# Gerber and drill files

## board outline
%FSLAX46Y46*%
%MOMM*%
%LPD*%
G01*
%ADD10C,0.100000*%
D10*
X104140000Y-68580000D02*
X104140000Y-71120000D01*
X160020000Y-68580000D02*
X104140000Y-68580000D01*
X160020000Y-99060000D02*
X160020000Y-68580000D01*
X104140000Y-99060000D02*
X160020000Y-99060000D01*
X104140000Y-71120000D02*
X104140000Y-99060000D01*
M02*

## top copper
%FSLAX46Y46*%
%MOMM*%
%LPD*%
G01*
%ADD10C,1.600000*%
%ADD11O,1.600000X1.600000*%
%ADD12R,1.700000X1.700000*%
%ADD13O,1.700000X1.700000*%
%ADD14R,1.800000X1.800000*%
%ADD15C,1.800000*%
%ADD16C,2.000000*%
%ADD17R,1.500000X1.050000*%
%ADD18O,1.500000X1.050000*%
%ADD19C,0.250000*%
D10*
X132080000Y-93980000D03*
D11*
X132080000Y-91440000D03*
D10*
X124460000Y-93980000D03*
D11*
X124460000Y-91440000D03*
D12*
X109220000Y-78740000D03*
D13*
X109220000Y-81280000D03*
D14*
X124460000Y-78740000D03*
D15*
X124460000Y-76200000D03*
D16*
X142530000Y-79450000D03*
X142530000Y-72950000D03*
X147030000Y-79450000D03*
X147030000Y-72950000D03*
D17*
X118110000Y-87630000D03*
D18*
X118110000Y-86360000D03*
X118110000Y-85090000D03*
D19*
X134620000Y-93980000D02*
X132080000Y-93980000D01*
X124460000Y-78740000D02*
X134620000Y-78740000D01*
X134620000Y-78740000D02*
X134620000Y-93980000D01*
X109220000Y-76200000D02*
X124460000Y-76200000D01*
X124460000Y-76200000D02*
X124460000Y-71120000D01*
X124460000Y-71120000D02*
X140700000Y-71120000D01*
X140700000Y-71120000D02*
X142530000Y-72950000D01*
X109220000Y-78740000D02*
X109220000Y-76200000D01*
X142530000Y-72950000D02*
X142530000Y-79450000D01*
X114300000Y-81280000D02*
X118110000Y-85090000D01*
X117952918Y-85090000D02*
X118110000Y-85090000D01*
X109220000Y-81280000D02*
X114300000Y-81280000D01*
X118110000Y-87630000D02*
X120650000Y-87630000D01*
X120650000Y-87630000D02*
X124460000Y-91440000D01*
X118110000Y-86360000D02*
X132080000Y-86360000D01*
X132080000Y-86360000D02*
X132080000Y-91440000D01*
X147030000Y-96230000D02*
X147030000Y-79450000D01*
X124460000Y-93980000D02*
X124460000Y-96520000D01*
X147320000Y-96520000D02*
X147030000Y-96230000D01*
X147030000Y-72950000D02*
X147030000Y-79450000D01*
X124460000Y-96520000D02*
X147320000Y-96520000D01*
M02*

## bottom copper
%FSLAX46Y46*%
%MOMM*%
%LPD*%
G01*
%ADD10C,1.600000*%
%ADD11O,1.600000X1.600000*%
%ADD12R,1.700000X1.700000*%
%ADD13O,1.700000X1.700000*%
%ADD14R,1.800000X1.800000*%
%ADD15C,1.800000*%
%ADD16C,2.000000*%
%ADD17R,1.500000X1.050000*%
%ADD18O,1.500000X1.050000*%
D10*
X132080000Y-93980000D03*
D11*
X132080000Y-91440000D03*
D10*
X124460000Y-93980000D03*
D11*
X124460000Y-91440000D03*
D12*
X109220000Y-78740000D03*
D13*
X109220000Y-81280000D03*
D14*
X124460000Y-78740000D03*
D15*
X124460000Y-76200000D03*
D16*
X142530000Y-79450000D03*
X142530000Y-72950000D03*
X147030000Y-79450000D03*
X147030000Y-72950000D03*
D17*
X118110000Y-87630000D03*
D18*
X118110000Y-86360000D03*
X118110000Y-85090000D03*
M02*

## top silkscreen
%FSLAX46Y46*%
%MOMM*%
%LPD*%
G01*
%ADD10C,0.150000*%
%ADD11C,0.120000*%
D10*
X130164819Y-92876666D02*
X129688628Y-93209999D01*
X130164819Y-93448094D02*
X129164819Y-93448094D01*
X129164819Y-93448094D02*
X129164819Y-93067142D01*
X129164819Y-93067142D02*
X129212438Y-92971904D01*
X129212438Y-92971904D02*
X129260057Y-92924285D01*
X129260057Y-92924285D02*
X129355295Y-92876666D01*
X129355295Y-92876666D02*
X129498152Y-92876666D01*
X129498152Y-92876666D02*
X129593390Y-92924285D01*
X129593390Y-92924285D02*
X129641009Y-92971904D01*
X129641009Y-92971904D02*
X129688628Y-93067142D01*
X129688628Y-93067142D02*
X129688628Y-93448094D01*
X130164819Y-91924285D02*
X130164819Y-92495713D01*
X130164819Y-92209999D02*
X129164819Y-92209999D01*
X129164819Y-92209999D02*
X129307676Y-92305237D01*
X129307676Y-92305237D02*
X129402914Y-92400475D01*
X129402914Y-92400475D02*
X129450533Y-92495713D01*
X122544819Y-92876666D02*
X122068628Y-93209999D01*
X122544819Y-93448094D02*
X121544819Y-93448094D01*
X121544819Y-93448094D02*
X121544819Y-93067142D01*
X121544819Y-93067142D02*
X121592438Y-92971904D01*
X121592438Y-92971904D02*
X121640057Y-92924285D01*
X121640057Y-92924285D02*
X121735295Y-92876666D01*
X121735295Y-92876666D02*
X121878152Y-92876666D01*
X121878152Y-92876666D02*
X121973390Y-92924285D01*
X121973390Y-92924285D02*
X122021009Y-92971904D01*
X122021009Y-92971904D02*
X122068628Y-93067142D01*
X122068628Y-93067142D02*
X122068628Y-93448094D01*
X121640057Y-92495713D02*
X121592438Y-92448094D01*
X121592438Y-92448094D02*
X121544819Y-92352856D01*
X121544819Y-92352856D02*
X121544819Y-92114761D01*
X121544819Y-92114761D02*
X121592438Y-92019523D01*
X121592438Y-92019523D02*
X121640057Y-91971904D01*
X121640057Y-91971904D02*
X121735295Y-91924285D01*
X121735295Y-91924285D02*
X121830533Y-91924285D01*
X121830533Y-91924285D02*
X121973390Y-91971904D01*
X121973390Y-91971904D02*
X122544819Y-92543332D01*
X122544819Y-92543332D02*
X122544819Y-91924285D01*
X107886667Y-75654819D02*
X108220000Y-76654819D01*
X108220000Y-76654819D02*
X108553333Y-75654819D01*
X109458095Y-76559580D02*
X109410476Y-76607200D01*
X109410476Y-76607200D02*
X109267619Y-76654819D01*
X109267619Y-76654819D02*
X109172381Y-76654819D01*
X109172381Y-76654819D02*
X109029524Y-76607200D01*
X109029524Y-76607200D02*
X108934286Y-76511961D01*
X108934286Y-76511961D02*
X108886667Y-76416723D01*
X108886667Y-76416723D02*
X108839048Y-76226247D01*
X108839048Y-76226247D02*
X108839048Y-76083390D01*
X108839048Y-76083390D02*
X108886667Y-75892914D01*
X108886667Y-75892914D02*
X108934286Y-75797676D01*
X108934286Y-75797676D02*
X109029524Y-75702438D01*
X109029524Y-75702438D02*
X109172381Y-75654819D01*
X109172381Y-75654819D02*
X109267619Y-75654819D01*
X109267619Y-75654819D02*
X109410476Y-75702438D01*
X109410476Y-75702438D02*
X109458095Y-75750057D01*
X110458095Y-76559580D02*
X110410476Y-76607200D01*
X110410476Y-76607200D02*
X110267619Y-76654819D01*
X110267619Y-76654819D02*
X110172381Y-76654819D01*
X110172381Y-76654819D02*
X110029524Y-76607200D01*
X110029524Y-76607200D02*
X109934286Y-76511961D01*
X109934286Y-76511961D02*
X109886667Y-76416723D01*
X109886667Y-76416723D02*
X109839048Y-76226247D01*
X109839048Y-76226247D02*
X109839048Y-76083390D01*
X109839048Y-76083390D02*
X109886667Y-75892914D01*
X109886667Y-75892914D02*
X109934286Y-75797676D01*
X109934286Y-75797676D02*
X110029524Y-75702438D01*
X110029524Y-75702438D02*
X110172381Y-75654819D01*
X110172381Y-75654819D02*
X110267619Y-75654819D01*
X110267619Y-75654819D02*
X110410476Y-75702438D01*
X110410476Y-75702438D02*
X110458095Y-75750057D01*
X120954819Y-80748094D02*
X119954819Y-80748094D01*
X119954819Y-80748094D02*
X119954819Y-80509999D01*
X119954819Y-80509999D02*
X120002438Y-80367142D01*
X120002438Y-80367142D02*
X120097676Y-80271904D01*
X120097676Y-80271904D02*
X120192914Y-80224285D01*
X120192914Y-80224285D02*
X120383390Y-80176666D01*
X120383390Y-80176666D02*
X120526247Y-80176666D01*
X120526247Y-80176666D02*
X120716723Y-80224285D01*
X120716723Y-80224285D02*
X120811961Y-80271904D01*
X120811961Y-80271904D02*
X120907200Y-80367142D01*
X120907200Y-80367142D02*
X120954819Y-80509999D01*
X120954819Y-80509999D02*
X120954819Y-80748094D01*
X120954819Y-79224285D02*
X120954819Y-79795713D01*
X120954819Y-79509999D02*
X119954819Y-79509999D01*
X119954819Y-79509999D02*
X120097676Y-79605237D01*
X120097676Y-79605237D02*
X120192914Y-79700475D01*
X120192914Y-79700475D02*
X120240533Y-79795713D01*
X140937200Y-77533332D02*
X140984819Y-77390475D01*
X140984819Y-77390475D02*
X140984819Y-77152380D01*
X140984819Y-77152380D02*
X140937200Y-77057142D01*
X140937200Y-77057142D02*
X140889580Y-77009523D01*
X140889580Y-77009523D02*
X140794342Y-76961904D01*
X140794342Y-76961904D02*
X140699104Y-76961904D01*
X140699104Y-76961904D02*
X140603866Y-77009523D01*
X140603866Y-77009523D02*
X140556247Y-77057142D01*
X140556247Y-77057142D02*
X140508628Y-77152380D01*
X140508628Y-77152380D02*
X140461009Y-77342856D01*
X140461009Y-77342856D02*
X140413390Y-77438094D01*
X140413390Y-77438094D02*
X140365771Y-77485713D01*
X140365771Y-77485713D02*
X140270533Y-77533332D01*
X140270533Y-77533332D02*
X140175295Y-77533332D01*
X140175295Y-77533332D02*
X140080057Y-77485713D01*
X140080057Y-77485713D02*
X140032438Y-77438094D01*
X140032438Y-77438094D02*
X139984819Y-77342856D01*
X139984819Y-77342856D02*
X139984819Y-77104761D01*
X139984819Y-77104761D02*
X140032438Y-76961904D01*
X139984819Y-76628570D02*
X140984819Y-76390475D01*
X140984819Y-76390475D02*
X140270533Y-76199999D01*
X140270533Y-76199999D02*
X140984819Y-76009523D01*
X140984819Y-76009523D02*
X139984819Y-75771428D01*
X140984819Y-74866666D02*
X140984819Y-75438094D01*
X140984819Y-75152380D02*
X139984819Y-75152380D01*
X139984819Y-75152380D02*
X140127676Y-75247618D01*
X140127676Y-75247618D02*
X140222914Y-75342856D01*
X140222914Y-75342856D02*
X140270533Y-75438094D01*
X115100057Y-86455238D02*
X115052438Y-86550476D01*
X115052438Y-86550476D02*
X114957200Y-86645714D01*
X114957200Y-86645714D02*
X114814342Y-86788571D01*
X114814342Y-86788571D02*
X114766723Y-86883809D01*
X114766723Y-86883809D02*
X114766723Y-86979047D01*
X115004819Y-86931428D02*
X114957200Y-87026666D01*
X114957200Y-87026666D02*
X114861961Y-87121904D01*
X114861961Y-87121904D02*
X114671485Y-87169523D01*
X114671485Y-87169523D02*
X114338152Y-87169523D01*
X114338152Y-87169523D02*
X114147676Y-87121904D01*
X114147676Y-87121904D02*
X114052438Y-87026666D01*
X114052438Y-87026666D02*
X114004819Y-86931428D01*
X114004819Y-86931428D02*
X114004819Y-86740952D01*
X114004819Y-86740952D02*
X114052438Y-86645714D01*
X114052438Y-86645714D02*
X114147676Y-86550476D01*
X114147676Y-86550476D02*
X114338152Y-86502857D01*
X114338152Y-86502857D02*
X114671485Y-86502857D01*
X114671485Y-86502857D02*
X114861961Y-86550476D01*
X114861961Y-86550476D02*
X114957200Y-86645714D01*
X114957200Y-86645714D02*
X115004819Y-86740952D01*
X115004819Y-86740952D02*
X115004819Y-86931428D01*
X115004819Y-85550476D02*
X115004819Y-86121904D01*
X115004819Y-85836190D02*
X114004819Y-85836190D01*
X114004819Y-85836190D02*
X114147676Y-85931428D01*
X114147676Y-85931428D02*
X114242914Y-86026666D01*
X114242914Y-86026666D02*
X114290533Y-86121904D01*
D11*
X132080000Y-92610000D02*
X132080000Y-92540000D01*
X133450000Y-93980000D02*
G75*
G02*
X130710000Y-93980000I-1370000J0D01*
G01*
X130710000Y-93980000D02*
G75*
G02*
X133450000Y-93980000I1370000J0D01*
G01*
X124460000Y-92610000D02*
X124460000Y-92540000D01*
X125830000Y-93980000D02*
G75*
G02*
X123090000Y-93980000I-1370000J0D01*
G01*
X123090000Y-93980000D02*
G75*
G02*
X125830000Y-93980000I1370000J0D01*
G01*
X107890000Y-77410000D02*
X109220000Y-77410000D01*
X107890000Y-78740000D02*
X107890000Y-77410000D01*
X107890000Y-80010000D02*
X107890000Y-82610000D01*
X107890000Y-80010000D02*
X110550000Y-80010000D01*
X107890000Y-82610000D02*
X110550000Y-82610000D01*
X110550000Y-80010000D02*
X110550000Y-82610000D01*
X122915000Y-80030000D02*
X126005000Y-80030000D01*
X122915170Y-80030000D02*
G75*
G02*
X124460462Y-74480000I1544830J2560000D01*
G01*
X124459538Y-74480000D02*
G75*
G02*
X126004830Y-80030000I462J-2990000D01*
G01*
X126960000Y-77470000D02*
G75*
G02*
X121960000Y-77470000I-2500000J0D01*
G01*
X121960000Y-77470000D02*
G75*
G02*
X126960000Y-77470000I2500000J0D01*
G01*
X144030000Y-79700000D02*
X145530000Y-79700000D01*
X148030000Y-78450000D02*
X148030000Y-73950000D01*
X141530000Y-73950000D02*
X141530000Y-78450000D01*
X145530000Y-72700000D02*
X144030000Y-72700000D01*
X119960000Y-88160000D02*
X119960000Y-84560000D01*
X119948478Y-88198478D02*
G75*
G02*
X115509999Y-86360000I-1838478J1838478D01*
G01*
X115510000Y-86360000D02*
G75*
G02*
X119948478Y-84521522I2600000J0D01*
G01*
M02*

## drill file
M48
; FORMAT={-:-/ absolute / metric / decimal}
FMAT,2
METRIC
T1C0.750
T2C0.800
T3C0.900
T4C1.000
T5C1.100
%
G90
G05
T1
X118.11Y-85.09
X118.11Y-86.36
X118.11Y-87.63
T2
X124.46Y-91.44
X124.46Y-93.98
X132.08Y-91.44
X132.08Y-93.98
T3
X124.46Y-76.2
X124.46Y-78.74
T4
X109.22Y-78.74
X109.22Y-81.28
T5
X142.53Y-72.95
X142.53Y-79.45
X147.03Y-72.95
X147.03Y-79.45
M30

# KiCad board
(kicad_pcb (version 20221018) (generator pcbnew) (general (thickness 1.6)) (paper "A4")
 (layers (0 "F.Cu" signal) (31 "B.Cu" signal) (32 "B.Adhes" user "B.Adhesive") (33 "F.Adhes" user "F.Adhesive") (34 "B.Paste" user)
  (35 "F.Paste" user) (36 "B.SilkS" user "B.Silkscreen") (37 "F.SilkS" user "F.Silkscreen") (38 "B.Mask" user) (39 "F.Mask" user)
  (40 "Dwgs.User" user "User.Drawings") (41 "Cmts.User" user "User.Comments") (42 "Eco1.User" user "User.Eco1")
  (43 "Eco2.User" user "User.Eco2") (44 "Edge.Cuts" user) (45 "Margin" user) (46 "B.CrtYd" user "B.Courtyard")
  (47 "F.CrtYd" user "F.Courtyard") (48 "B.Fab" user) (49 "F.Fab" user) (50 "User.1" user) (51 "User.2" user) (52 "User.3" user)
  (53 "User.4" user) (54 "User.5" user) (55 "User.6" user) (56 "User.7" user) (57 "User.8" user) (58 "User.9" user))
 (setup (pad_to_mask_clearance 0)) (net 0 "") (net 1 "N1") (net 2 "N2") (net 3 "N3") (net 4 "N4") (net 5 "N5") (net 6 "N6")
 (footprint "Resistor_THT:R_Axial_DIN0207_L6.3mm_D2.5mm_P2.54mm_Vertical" (layer "F.Cu") (at 132.08 93.98 90)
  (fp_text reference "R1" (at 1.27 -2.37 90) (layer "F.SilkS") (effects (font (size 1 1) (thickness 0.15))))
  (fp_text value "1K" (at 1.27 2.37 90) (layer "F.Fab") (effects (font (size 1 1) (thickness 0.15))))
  (fp_line (start 1.37 0) (end 1.44 0) (stroke (width 0.12) (type solid)) (layer "F.SilkS"))
  (fp_circle (center 0 0) (end 1.37 0) (stroke (width 0.12) (type solid)) (fill none) (layer "F.SilkS"))
  (pad "1" thru_hole circle (at 0 0 90) (size 1.6 1.6) (drill 0.8) (layers "*.Cu" "*.Mask") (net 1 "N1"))
  (pad "2" thru_hole oval (at 2.54 0 90) (size 1.6 1.6) (drill 0.8) (layers "*.Cu" "*.Mask") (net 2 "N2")))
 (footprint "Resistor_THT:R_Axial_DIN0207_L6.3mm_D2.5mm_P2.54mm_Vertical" (layer "F.Cu") (at 124.46 93.98 90)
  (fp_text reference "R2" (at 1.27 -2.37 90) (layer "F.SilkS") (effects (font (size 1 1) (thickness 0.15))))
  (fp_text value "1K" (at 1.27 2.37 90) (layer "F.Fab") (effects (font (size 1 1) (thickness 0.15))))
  (fp_line (start 1.37 0) (end 1.44 0) (stroke (width 0.12) (type solid)) (layer "F.SilkS"))
  (fp_circle (center 0 0) (end 1.37 0) (stroke (width 0.12) (type solid)) (fill none) (layer "F.SilkS"))
  (pad "1" thru_hole circle (at 0 0 90) (size 1.6 1.6) (drill 0.8) (layers "*.Cu" "*.Mask") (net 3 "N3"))
  (pad "2" thru_hole oval (at 2.54 0 90) (size 1.6 1.6) (drill 0.8) (layers "*.Cu" "*.Mask") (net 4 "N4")))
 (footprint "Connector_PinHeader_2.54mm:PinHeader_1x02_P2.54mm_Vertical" (layer "F.Cu") (at 109.22 78.74)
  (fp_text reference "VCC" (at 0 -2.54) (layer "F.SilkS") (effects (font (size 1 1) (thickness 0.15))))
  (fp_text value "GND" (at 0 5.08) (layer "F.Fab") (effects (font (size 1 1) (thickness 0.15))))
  (fp_line (start -1.33 -1.33) (end 0 -1.33) (stroke (width 0.12) (type solid)) (layer "F.SilkS"))
  (fp_line (start -1.33 0) (end -1.33 -1.33) (stroke (width 0.12) (type solid)) (layer "F.SilkS"))
  (fp_line (start -1.33 1.27) (end -1.33 3.87) (stroke (width 0.12) (type solid)) (layer "F.SilkS"))
  (fp_line (start -1.33 1.27) (end 1.33 1.27) (stroke (width 0.12) (type solid)) (layer "F.SilkS"))
  (fp_line (start -1.33 3.87) (end 1.33 3.87) (stroke (width 0.12) (type solid)) (layer "F.SilkS"))
  (fp_line (start 1.33 1.27) (end 1.33 3.87) (stroke (width 0.12) (type solid)) (layer "F.SilkS"))
  (pad "1" thru_hole rect (at 0 0) (size 1.7 1.7) (drill 1) (layers "*.Cu" "*.Mask") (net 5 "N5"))
  (pad "2" thru_hole oval (at 0 2.54) (size 1.7 1.7) (drill 1) (layers "*.Cu" "*.Mask") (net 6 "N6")))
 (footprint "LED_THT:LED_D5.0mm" (layer "F.Cu") (at 124.46 78.74 90)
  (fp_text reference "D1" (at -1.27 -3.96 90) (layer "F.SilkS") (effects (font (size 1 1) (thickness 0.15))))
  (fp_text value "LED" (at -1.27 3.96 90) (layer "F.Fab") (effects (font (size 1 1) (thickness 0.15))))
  (fp_line (start -1.29 -1.545) (end -1.29 1.545) (stroke (width 0.12) (type solid)) (layer "F.SilkS"))
  (fp_arc (start -1.29 -1.54483) (mid 2.072002 -2.880433) (end 4.26 0.000462) (stroke (width 0.12) (type solid)) (layer "F.SilkS"))
  (fp_arc (start 4.26 -0.000462) (mid 2.072002 2.880433) (end -1.29 1.54483) (stroke (width 0.12) (type solid)) (layer "F.SilkS"))
  (fp_circle (center 1.27 0) (end 3.77 0) (stroke (width 0.12) (type solid)) (fill none) (layer "F.SilkS"))
  (pad "1" thru_hole rect (at 0 0 90) (size 1.8 1.8) (drill 0.9) (layers "*.Cu" "*.Mask") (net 1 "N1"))
  (pad "2" thru_hole circle (at 2.54 0 90) (size 1.8 1.8) (drill 0.9) (layers "*.Cu" "*.Mask") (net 5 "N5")))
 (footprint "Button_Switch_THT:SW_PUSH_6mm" (layer "F.Cu") (at 142.53 79.45 90)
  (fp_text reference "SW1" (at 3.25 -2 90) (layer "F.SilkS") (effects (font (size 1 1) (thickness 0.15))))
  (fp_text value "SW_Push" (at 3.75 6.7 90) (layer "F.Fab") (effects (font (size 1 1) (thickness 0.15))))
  (fp_line (start -0.25 1.5) (end -0.25 3) (stroke (width 0.12) (type solid)) (layer "F.SilkS"))
  (fp_line (start 1 5.5) (end 5.5 5.5) (stroke (width 0.12) (type solid)) (layer "F.SilkS"))
  (fp_line (start 5.5 -1) (end 1 -1) (stroke (width 0.12) (type solid)) (layer "F.SilkS"))
  (fp_line (start 6.75 3) (end 6.75 1.5) (stroke (width 0.12) (type solid)) (layer "F.SilkS"))
  (pad "1" thru_hole circle (at 0 0 180) (size 2 2) (drill 1.1) (layers "*.Cu" "*.Mask") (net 5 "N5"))
  (pad "1" thru_hole circle (at 6.5 0 180) (size 2 2) (drill 1.1) (layers "*.Cu" "*.Mask") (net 5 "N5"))
  (pad "2" thru_hole circle (at 0 4.5 180) (size 2 2) (drill 1.1) (layers "*.Cu" "*.Mask") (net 3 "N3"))
  (pad "2" thru_hole circle (at 6.5 4.5 180) (size 2 2) (drill 1.1) (layers "*.Cu" "*.Mask") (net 3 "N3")))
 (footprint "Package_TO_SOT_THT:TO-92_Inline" (layer "F.Cu") (at 118.11 87.63 90)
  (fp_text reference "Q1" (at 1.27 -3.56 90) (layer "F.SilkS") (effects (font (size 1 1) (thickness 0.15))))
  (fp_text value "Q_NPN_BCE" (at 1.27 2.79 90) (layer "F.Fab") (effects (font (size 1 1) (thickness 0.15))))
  (fp_line (start -0.53 1.85) (end 3.07 1.85) (stroke (width 0.12) (type solid)) (layer "F.SilkS"))
  (fp_arc (start -0.568478 1.838478) (mid -1.132087 -0.994977) (end 1.27 -2.6) (stroke (width 0.12) (type solid)) (layer "F.SilkS"))
  (fp_arc (start 1.27 -2.6) (mid 3.672087 -0.994977) (end 3.108478 1.838478) (stroke (width 0.12) (type solid)) (layer "F.SilkS"))
  (pad "1" thru_hole rect (at 0 0 90) (size 1.05 1.5) (drill 0.75) (layers "*.Cu" "*.Mask") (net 4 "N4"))
  (pad "2" thru_hole oval (at 1.27 0 90) (size 1.05 1.5) (drill 0.75) (layers "*.Cu" "*.Mask") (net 2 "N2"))
  (pad "3" thru_hole oval (at 2.54 0 90) (size 1.05 1.5) (drill 0.75) (layers "*.Cu" "*.Mask") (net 6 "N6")))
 (gr_line (start 104.14 68.58) (end 104.14 71.12) (stroke (width 0.1) (type default)) (layer "Edge.Cuts"))
 (gr_line (start 160.02 68.58) (end 104.14 68.58) (stroke (width 0.1) (type default)) (layer "Edge.Cuts"))
 (gr_line (start 160.02 99.06) (end 160.02 68.58) (stroke (width 0.1) (type default)) (layer "Edge.Cuts"))
 (gr_line (start 104.14 99.06) (end 160.02 99.06) (stroke (width 0.1) (type default)) (layer "Edge.Cuts"))
 (gr_line (start 104.14 71.12) (end 104.14 99.06) (stroke (width 0.1) (type default)) (layer "Edge.Cuts"))
 (segment (start 134.62 93.98) (end 132.08 93.98) (width 0.25) (layer "F.Cu") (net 1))
 (segment (start 124.46 78.74) (end 134.62 78.74) (width 0.25) (layer "F.Cu") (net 1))
 (segment (start 134.62 78.74) (end 134.62 93.98) (width 0.25) (layer "F.Cu") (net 1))
 (segment (start 109.22 76.2) (end 124.46 76.2) (width 0.25) (layer "F.Cu") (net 5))
 (segment (start 124.46 76.2) (end 124.46 71.12) (width 0.25) (layer "F.Cu") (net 5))
 (segment (start 124.46 71.12) (end 140.7 71.12) (width 0.25) (layer "F.Cu") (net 5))
 (segment (start 140.7 71.12) (end 142.53 72.95) (width 0.25) (layer "F.Cu") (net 5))
 (segment (start 109.22 78.74) (end 109.22 76.2) (width 0.25) (layer "F.Cu") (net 5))
 (segment (start 142.53 72.95) (end 142.53 79.45) (width 0.25) (layer "F.Cu") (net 5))
 (segment (start 114.3 81.28) (end 118.11 85.09) (width 0.25) (layer "F.Cu") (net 6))
 (segment (start 117.952918 85.09) (end 118.11 85.09) (width 0.25) (layer "F.Cu") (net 6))
 (segment (start 109.22 81.28) (end 114.3 81.28) (width 0.25) (layer "F.Cu") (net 6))
 (segment (start 118.11 87.63) (end 120.65 87.63) (width 0.25) (layer "F.Cu") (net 4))
 (segment (start 120.65 87.63) (end 124.46 91.44) (width 0.25) (layer "F.Cu") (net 4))
 (segment (start 118.11 86.36) (end 132.08 86.36) (width 0.25) (layer "F.Cu") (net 2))
 (segment (start 132.08 86.36) (end 132.08 91.44) (width 0.25) (layer "F.Cu") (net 2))
 (segment (start 147.03 96.23) (end 147.03 79.45) (width 0.25) (layer "F.Cu") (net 3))
 (segment (start 124.46 93.98) (end 124.46 96.52) (width 0.25) (layer "F.Cu") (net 3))
 (segment (start 147.32 96.52) (end 147.03 96.23) (width 0.25) (layer "F.Cu") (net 3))
 (segment (start 147.03 72.95) (end 147.03 79.45) (width 0.25) (layer "F.Cu") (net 3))
 (segment (start 124.46 96.52) (end 147.32 96.52) (width 0.25) (layer "F.Cu") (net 3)))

